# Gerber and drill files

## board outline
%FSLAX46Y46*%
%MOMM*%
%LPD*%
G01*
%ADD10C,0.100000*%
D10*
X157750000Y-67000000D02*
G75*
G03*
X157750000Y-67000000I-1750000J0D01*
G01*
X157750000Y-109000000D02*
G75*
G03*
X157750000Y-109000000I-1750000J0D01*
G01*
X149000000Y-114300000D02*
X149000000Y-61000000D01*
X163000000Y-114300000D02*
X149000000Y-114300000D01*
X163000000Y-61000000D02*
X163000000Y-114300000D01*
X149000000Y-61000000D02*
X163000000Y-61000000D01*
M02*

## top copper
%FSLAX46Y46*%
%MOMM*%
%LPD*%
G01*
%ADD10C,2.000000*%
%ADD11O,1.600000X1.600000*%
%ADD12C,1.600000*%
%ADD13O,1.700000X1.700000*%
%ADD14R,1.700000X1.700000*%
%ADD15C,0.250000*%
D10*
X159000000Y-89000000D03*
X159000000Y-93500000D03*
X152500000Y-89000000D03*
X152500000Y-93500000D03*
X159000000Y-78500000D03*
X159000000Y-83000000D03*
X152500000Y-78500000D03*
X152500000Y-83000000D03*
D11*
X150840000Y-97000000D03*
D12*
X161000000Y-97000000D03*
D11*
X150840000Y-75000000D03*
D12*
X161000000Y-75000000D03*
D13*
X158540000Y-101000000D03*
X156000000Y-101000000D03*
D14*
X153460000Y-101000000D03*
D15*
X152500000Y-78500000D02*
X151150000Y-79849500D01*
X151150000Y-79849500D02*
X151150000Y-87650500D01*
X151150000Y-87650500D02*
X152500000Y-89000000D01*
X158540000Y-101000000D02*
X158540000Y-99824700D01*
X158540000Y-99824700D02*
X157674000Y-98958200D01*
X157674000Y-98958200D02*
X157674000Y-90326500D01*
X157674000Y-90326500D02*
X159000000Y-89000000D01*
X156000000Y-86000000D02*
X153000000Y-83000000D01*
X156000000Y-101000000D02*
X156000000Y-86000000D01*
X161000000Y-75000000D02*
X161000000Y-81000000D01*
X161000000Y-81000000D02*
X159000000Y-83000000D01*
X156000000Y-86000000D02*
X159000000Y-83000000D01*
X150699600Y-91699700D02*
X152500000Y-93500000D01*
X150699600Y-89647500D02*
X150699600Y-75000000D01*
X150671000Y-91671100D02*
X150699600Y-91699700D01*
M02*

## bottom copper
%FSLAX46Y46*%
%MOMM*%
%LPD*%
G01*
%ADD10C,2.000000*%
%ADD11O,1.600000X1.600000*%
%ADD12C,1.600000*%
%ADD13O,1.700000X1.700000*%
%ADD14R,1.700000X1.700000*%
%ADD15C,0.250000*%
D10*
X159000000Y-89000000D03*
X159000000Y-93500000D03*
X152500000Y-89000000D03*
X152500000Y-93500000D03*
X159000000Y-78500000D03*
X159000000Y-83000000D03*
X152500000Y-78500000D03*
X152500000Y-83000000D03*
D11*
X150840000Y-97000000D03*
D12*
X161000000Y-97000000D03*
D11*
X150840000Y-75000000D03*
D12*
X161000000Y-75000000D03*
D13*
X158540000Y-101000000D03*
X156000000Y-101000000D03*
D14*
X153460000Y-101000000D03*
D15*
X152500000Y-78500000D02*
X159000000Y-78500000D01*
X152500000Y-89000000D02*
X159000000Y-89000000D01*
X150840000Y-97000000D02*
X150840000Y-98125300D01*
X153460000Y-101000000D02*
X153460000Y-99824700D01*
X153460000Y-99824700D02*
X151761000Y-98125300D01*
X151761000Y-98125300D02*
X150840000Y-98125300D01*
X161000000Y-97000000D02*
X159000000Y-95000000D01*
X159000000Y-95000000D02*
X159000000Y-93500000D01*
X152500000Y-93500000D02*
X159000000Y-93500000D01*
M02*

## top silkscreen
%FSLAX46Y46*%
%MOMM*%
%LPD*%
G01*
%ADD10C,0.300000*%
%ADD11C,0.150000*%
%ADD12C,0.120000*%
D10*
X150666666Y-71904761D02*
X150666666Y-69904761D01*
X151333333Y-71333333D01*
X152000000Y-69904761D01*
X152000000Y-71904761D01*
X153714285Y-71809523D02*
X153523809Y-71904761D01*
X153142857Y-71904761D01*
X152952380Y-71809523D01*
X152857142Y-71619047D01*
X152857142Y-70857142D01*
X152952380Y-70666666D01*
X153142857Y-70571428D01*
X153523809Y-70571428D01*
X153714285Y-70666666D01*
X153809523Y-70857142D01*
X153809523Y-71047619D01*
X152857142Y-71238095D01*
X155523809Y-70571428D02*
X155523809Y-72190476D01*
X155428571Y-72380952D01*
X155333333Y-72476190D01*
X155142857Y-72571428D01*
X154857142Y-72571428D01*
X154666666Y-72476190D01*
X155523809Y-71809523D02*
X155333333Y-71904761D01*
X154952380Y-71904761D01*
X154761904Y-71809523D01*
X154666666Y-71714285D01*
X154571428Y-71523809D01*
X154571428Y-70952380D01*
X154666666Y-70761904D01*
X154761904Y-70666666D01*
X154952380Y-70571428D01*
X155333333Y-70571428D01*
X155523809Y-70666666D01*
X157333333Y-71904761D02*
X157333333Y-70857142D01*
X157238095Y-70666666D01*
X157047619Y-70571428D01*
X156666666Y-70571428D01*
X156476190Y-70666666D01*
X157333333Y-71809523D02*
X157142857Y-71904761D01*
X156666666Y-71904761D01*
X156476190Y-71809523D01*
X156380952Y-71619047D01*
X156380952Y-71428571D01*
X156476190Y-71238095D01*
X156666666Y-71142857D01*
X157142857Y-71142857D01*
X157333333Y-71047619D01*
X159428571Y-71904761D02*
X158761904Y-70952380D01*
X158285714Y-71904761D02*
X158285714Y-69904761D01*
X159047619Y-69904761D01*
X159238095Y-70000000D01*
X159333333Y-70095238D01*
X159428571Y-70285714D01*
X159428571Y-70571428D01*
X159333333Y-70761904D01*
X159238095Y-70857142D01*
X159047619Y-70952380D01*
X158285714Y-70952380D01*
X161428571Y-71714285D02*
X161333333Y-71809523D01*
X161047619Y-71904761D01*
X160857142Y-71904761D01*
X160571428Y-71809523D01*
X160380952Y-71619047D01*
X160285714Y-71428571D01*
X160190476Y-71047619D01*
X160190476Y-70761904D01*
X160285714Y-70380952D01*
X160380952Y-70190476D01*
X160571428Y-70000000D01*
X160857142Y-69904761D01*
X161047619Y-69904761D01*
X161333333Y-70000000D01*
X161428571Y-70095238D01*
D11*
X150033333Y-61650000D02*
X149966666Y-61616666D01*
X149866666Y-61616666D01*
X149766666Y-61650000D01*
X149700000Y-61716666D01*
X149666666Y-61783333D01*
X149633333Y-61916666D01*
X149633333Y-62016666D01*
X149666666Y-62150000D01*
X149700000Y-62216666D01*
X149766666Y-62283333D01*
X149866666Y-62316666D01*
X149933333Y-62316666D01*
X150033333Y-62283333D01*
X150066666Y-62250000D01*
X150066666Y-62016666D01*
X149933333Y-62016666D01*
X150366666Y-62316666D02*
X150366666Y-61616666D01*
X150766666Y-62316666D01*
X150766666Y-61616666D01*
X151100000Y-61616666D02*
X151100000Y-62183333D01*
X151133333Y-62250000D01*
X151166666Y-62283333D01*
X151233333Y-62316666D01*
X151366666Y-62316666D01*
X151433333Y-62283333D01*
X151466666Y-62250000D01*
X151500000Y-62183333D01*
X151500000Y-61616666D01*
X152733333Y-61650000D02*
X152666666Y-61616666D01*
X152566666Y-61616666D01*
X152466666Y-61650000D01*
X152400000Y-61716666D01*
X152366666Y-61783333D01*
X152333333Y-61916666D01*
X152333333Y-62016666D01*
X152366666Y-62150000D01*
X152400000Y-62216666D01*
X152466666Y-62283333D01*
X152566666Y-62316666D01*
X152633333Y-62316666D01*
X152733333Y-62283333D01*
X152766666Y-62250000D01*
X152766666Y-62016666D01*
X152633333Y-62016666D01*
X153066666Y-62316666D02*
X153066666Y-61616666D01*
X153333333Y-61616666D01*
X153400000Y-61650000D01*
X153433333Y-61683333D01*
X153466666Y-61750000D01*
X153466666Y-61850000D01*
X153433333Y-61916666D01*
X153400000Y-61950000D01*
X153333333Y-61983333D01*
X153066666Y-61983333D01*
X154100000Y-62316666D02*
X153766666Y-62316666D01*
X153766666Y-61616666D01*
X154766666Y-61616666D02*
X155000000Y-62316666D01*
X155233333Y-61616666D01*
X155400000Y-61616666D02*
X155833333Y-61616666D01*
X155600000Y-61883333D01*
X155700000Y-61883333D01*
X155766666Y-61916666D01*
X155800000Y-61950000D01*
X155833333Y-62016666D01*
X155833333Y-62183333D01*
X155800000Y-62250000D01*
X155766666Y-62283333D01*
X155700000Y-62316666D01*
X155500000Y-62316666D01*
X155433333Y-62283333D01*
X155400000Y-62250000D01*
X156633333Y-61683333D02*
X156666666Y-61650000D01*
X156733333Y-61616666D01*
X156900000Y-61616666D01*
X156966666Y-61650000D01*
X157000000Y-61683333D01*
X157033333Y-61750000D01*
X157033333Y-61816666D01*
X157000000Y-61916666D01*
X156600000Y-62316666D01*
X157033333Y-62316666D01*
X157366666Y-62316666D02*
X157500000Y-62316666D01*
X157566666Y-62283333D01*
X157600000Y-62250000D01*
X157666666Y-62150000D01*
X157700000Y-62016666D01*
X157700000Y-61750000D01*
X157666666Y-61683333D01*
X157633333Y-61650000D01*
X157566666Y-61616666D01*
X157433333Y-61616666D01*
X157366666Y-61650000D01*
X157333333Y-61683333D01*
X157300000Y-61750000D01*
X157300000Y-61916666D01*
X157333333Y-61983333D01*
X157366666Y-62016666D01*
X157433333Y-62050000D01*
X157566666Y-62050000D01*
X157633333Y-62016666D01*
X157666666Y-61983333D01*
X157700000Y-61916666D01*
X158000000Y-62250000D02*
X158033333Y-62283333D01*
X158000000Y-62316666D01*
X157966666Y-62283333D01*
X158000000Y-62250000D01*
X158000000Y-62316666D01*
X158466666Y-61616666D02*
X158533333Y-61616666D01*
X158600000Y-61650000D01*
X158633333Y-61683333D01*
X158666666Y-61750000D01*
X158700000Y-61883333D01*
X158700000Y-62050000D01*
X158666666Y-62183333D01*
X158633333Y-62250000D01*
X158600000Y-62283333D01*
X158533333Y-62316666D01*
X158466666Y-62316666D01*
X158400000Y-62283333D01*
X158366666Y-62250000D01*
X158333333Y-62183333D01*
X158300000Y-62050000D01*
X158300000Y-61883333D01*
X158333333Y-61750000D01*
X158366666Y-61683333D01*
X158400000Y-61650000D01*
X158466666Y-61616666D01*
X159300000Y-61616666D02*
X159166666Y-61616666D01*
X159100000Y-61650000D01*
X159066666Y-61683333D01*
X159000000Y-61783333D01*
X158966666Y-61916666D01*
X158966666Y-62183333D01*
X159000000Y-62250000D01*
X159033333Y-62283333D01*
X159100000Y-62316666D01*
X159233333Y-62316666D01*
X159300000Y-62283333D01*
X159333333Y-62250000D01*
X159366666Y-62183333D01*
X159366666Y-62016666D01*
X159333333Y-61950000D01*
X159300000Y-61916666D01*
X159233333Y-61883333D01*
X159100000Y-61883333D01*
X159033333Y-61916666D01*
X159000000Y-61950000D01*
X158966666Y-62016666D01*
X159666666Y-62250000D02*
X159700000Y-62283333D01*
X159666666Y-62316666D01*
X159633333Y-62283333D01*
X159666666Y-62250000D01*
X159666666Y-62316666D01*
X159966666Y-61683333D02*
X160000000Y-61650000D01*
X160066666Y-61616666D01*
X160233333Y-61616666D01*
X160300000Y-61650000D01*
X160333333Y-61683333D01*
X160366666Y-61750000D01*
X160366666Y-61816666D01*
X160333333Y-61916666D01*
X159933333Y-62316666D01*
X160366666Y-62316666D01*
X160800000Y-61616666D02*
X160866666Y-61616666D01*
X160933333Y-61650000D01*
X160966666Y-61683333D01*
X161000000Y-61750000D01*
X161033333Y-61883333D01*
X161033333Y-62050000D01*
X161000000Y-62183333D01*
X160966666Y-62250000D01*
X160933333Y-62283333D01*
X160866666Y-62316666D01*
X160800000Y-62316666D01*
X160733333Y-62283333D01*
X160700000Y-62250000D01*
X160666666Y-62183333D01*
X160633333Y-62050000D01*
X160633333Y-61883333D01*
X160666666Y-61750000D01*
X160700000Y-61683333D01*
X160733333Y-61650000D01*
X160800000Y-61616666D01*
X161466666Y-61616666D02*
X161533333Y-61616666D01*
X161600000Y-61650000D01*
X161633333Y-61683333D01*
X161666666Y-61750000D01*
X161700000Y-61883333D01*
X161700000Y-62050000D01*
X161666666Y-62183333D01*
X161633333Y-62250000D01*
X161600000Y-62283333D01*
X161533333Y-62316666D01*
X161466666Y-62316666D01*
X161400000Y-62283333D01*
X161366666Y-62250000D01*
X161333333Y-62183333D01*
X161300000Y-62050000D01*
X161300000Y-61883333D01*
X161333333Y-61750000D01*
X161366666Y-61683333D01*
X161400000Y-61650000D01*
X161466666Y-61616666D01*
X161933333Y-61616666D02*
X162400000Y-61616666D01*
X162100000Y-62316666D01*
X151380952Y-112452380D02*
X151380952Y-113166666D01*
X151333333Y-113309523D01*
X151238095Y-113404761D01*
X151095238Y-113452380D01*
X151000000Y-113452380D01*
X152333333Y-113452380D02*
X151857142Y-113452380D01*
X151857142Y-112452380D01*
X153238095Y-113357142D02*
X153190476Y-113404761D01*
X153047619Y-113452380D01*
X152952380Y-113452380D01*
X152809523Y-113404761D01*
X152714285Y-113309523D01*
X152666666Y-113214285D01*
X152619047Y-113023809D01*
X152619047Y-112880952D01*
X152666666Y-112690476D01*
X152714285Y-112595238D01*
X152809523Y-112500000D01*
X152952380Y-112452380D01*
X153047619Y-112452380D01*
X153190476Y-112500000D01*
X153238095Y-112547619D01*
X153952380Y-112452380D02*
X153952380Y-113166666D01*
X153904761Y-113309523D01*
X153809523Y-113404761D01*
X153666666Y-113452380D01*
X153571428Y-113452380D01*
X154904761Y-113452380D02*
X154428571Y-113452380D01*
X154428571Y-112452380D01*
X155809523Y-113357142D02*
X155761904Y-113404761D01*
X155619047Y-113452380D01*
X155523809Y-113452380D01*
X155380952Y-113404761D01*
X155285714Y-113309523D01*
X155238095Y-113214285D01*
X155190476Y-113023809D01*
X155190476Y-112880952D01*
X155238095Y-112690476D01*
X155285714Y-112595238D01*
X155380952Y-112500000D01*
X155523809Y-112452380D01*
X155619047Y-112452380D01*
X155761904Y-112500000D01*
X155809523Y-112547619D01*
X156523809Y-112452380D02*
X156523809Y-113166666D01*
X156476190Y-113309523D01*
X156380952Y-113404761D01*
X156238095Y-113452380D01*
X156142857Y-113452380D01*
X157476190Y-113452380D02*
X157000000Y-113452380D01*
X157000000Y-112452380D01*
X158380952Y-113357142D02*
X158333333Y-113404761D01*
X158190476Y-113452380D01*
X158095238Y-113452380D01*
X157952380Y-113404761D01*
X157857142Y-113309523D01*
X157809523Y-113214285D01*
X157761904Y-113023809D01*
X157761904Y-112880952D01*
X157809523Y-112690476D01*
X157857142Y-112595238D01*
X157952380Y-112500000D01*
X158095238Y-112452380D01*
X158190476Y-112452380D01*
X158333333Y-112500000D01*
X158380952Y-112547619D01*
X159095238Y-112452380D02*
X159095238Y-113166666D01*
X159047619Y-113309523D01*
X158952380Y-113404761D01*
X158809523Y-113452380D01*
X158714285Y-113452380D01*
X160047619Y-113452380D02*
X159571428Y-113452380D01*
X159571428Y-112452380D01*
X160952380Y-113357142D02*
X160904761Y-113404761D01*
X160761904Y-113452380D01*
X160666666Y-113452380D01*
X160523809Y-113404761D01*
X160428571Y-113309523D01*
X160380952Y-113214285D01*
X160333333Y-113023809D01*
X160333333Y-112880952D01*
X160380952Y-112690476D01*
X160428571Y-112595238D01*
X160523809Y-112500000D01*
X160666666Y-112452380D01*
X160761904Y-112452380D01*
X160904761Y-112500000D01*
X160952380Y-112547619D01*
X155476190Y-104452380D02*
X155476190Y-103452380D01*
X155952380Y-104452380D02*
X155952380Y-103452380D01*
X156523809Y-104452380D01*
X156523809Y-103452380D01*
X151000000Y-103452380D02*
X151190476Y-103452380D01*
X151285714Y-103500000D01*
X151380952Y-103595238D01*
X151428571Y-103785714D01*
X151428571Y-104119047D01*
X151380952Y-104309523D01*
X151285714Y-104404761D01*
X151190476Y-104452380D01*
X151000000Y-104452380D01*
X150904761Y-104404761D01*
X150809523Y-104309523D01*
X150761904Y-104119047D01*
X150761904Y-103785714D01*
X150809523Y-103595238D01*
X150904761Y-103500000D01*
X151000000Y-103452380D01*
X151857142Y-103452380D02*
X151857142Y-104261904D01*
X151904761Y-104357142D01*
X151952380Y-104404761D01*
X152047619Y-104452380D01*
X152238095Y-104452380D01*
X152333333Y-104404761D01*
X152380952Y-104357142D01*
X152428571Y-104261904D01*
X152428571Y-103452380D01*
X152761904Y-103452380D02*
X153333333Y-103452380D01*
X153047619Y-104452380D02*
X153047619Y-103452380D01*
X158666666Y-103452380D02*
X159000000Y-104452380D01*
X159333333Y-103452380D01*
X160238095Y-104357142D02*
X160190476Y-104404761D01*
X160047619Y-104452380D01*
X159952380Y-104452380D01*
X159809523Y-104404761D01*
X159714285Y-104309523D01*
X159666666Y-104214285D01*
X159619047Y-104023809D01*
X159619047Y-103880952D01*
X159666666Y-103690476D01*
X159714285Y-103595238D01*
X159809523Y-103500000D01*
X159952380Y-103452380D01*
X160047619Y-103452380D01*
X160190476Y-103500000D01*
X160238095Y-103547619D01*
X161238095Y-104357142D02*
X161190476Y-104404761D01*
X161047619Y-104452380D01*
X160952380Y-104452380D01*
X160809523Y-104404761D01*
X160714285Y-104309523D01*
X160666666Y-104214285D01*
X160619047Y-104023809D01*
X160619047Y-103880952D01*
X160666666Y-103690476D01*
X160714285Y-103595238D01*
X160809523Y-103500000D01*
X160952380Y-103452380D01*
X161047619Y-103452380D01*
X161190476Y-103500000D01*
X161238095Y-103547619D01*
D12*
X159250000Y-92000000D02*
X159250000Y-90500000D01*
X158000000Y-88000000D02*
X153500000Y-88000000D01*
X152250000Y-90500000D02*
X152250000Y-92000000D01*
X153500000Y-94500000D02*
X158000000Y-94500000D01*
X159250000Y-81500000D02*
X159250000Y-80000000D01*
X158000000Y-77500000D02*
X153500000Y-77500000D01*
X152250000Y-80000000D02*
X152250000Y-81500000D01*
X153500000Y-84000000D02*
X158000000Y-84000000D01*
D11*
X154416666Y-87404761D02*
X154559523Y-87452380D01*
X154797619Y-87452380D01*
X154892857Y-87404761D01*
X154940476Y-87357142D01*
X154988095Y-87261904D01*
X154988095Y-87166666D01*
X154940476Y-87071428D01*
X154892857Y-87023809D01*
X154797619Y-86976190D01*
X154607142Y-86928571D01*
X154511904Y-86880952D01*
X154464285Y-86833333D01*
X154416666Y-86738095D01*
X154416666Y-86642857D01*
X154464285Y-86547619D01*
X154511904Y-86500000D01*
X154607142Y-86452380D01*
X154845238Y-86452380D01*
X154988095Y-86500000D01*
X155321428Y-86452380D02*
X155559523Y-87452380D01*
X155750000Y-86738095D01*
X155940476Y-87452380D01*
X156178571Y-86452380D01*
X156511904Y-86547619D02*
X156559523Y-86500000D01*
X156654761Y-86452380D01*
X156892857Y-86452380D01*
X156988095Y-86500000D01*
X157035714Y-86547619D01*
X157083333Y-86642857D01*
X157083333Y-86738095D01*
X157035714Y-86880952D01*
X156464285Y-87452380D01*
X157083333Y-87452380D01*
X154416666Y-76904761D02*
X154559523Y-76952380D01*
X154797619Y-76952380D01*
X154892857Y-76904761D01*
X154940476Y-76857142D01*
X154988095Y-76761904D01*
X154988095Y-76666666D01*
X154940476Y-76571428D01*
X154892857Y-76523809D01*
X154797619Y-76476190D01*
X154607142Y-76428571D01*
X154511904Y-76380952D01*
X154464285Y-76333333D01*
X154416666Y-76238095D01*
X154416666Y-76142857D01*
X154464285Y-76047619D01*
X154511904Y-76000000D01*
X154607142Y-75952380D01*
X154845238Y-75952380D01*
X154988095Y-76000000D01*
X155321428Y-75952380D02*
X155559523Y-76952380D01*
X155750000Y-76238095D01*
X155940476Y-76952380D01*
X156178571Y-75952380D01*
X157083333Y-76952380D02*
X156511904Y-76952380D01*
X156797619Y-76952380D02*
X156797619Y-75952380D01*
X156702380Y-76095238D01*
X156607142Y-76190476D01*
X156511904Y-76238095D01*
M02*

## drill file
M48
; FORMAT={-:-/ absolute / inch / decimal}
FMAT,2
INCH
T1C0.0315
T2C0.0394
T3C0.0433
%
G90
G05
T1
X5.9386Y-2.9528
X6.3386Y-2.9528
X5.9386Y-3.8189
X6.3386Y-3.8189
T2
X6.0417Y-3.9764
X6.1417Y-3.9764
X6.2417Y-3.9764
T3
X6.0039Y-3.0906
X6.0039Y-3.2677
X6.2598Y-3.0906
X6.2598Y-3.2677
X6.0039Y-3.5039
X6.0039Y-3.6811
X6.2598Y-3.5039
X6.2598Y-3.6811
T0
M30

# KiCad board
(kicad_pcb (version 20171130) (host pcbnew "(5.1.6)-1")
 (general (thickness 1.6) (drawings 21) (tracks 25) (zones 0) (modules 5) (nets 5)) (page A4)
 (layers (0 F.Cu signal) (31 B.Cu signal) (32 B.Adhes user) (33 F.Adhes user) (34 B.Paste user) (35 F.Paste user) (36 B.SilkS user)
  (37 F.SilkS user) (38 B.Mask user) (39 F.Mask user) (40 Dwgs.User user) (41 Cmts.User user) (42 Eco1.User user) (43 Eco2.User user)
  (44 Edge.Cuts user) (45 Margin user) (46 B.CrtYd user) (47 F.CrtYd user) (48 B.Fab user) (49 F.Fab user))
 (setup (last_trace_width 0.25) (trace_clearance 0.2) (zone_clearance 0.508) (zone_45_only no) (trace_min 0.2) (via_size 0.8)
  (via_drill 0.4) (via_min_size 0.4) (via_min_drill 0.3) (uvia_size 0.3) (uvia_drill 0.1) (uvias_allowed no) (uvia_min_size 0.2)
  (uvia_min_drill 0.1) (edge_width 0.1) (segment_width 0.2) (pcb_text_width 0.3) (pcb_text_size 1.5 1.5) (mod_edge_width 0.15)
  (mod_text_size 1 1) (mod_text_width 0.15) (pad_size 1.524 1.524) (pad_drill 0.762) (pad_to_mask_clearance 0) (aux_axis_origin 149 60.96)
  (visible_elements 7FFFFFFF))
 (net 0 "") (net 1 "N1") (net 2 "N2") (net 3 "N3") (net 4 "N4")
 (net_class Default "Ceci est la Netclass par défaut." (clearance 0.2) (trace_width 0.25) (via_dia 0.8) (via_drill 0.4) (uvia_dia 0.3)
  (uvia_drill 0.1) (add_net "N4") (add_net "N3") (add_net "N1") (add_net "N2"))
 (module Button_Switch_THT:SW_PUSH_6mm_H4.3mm (layer F.Cu) (at 152.5 89)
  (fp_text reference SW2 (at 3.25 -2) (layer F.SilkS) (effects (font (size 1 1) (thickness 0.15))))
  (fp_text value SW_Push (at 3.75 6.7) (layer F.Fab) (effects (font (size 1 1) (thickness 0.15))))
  (fp_line (start 1 5.5) (end 5.5 5.5) (layer F.SilkS) (width 0.12))
  (fp_line (start -0.25 1.5) (end -0.25 3) (layer F.SilkS) (width 0.12))
  (fp_line (start 5.5 -1) (end 1 -1) (layer F.SilkS) (width 0.12))
  (fp_line (start 6.75 3) (end 6.75 1.5) (layer F.SilkS) (width 0.12))
  (pad 1 thru_hole circle (at 6.5 0 90) (size 2 2) (drill 1.1) (layers *.Cu *.Mask) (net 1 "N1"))
  (pad 2 thru_hole circle (at 6.5 4.5 90) (size 2 2) (drill 1.1) (layers *.Cu *.Mask) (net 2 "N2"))
  (pad 1 thru_hole circle (at 0 0 90) (size 2 2) (drill 1.1) (layers *.Cu *.Mask) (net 1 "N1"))
  (pad 2 thru_hole circle (at 0 4.5 90) (size 2 2) (drill 1.1) (layers *.Cu *.Mask) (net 2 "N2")))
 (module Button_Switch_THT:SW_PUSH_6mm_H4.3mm (layer F.Cu) (at 152.5 78.5)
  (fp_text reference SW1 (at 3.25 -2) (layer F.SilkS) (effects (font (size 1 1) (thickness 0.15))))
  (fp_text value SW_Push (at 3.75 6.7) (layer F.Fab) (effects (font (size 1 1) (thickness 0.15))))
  (fp_line (start 1 5.5) (end 5.5 5.5) (layer F.SilkS) (width 0.12))
  (fp_line (start -0.25 1.5) (end -0.25 3) (layer F.SilkS) (width 0.12))
  (fp_line (start 5.5 -1) (end 1 -1) (layer F.SilkS) (width 0.12))
  (fp_line (start 6.75 3) (end 6.75 1.5) (layer F.SilkS) (width 0.12))
  (pad 1 thru_hole circle (at 6.5 0 90) (size 2 2) (drill 1.1) (layers *.Cu *.Mask) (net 1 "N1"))
  (pad 2 thru_hole circle (at 6.5 4.5 90) (size 2 2) (drill 1.1) (layers *.Cu *.Mask) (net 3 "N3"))
  (pad 1 thru_hole circle (at 0 0 90) (size 2 2) (drill 1.1) (layers *.Cu *.Mask) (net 1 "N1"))
  (pad 2 thru_hole circle (at 0 4.5 90) (size 2 2) (drill 1.1) (layers *.Cu *.Mask) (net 3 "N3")))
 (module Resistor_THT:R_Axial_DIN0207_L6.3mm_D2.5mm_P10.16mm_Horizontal (layer B.Cu) (at 161 97 180)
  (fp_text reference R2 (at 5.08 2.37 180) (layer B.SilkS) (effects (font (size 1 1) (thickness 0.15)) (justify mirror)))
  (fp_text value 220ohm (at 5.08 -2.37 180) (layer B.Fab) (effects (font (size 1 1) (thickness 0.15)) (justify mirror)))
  (pad 2 thru_hole oval (at 10.16 0 180) (size 1.6 1.6) (drill 0.8) (layers *.Cu *.Mask) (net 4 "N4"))
  (pad 1 thru_hole circle (at 0 0 180) (size 1.6 1.6) (drill 0.8) (layers *.Cu *.Mask) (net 2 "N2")))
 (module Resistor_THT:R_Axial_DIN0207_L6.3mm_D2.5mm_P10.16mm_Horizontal (layer B.Cu) (at 161 75 180)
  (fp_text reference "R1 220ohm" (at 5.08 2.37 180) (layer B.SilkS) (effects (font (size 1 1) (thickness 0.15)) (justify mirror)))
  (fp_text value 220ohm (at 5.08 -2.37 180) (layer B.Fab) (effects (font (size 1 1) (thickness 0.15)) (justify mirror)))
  (pad 2 thru_hole oval (at 10.16 0 180) (size 1.6 1.6) (drill 0.8) (layers *.Cu *.Mask) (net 2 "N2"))
  (pad 1 thru_hole circle (at 0 0 180) (size 1.6 1.6) (drill 0.8) (layers *.Cu *.Mask) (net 3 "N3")))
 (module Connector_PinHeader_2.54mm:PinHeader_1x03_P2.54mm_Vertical (layer B.Cu) (at 153.46 101 270)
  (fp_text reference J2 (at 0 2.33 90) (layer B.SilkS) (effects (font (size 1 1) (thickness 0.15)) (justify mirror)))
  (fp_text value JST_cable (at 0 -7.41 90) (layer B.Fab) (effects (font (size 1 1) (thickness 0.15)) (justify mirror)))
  (pad 3 thru_hole oval (at 0 -5.08 270) (size 1.7 1.7) (drill 1) (layers *.Cu *.Mask) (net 1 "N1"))
  (pad 2 thru_hole oval (at 0 -2.54 270) (size 1.7 1.7) (drill 1) (layers *.Cu *.Mask) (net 3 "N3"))
  (pad 1 thru_hole rect (at 0 0 270) (size 1.7 1.7) (drill 1) (layers *.Cu *.Mask) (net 4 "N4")))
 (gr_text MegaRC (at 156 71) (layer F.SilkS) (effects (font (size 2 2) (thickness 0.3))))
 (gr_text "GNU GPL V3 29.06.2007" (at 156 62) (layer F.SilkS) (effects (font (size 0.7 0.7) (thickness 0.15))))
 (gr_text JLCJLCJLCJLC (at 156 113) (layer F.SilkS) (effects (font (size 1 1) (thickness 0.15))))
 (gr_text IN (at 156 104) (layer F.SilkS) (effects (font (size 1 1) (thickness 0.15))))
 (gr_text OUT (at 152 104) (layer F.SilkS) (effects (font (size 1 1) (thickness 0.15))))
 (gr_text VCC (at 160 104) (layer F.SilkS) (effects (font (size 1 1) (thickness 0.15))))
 (gr_circle (center 156 67) (end 157.75 67) (layer Edge.Cuts) (width 0.1))
 (gr_circle (center 156 109) (end 157.75 109) (layer Edge.Cuts) (width 0.1))
 (gr_line (start 149 114.3) (end 149 61) (layer Edge.Cuts) (width 0.1))
 (gr_line (start 163 114.3) (end 149 114.3) (layer Edge.Cuts) (width 0.1))
 (gr_line (start 163 61) (end 163 114.3) (layer Edge.Cuts) (width 0.1))
 (gr_line (start 149 61) (end 163 61) (layer Edge.Cuts) (width 0.1))
 (segment (start 152.5 78.5) (end 159 78.5) (width 0.25) (layer B.Cu) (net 1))
 (segment (start 152.5 78.5) (end 151.15 79.8495) (width 0.25) (layer F.Cu) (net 1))
 (segment (start 151.15 79.8495) (end 151.15 87.6505) (width 0.25) (layer F.Cu) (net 1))
 (segment (start 151.15 87.6505) (end 152.5 89) (width 0.25) (layer F.Cu) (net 1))
 (segment (start 152.5 89) (end 159 89) (width 0.25) (layer B.Cu) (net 1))
 (segment (start 158.54 101) (end 158.54 99.8247) (width 0.25) (layer F.Cu) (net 1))
 (segment (start 158.54 99.8247) (end 157.674 98.9582) (width 0.25) (layer F.Cu) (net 1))
 (segment (start 157.674 98.9582) (end 157.674 90.3265) (width 0.25) (layer F.Cu) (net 1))
 (segment (start 157.674 90.3265) (end 159 89) (width 0.25) (layer F.Cu) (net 1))
 (segment (start 156 86) (end 153 83) (width 0.25) (layer F.Cu) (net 3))
 (segment (start 156 101) (end 156 86) (width 0.25) (layer F.Cu) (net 3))
 (segment (start 161 75) (end 161 81) (width 0.25) (layer F.Cu) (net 3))
 (segment (start 161 81) (end 159 83) (width 0.25) (layer F.Cu) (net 3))
 (segment (start 156 86) (end 159 83) (width 0.25) (layer F.Cu) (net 3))
 (segment (start 150.84 97) (end 150.84 98.1253) (width 0.25) (layer B.Cu) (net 4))
 (segment (start 153.46 101) (end 153.46 99.8247) (width 0.25) (layer B.Cu) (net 4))
 (segment (start 153.46 99.8247) (end 151.761 98.1253) (width 0.25) (layer B.Cu) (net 4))
 (segment (start 151.761 98.1253) (end 150.84 98.1253) (width 0.25) (layer B.Cu) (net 4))
 (segment (start 161 97) (end 159 95) (width 0.25) (layer B.Cu) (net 2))
 (segment (start 159 95) (end 159 93.5) (width 0.25) (layer B.Cu) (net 2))
 (segment (start 152.5 93.5) (end 159 93.5) (width 0.25) (layer B.Cu) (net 2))
 (segment (start 150.6996 91.6997) (end 152.5 93.5) (width 0.25) (layer F.Cu) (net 2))
 (segment (start 150.671 91.6711) (end 150.6996 91.6997) (width 0.25) (layer F.Cu) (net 2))
 (segment (start 150.6996 75) (end 150.6996 91.6425) (width 0.25) (layer F.Cu) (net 2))
 (segment (start 150.6996 91.6425) (end 150.671 91.6711) (width 0.25) (layer F.Cu) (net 2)))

